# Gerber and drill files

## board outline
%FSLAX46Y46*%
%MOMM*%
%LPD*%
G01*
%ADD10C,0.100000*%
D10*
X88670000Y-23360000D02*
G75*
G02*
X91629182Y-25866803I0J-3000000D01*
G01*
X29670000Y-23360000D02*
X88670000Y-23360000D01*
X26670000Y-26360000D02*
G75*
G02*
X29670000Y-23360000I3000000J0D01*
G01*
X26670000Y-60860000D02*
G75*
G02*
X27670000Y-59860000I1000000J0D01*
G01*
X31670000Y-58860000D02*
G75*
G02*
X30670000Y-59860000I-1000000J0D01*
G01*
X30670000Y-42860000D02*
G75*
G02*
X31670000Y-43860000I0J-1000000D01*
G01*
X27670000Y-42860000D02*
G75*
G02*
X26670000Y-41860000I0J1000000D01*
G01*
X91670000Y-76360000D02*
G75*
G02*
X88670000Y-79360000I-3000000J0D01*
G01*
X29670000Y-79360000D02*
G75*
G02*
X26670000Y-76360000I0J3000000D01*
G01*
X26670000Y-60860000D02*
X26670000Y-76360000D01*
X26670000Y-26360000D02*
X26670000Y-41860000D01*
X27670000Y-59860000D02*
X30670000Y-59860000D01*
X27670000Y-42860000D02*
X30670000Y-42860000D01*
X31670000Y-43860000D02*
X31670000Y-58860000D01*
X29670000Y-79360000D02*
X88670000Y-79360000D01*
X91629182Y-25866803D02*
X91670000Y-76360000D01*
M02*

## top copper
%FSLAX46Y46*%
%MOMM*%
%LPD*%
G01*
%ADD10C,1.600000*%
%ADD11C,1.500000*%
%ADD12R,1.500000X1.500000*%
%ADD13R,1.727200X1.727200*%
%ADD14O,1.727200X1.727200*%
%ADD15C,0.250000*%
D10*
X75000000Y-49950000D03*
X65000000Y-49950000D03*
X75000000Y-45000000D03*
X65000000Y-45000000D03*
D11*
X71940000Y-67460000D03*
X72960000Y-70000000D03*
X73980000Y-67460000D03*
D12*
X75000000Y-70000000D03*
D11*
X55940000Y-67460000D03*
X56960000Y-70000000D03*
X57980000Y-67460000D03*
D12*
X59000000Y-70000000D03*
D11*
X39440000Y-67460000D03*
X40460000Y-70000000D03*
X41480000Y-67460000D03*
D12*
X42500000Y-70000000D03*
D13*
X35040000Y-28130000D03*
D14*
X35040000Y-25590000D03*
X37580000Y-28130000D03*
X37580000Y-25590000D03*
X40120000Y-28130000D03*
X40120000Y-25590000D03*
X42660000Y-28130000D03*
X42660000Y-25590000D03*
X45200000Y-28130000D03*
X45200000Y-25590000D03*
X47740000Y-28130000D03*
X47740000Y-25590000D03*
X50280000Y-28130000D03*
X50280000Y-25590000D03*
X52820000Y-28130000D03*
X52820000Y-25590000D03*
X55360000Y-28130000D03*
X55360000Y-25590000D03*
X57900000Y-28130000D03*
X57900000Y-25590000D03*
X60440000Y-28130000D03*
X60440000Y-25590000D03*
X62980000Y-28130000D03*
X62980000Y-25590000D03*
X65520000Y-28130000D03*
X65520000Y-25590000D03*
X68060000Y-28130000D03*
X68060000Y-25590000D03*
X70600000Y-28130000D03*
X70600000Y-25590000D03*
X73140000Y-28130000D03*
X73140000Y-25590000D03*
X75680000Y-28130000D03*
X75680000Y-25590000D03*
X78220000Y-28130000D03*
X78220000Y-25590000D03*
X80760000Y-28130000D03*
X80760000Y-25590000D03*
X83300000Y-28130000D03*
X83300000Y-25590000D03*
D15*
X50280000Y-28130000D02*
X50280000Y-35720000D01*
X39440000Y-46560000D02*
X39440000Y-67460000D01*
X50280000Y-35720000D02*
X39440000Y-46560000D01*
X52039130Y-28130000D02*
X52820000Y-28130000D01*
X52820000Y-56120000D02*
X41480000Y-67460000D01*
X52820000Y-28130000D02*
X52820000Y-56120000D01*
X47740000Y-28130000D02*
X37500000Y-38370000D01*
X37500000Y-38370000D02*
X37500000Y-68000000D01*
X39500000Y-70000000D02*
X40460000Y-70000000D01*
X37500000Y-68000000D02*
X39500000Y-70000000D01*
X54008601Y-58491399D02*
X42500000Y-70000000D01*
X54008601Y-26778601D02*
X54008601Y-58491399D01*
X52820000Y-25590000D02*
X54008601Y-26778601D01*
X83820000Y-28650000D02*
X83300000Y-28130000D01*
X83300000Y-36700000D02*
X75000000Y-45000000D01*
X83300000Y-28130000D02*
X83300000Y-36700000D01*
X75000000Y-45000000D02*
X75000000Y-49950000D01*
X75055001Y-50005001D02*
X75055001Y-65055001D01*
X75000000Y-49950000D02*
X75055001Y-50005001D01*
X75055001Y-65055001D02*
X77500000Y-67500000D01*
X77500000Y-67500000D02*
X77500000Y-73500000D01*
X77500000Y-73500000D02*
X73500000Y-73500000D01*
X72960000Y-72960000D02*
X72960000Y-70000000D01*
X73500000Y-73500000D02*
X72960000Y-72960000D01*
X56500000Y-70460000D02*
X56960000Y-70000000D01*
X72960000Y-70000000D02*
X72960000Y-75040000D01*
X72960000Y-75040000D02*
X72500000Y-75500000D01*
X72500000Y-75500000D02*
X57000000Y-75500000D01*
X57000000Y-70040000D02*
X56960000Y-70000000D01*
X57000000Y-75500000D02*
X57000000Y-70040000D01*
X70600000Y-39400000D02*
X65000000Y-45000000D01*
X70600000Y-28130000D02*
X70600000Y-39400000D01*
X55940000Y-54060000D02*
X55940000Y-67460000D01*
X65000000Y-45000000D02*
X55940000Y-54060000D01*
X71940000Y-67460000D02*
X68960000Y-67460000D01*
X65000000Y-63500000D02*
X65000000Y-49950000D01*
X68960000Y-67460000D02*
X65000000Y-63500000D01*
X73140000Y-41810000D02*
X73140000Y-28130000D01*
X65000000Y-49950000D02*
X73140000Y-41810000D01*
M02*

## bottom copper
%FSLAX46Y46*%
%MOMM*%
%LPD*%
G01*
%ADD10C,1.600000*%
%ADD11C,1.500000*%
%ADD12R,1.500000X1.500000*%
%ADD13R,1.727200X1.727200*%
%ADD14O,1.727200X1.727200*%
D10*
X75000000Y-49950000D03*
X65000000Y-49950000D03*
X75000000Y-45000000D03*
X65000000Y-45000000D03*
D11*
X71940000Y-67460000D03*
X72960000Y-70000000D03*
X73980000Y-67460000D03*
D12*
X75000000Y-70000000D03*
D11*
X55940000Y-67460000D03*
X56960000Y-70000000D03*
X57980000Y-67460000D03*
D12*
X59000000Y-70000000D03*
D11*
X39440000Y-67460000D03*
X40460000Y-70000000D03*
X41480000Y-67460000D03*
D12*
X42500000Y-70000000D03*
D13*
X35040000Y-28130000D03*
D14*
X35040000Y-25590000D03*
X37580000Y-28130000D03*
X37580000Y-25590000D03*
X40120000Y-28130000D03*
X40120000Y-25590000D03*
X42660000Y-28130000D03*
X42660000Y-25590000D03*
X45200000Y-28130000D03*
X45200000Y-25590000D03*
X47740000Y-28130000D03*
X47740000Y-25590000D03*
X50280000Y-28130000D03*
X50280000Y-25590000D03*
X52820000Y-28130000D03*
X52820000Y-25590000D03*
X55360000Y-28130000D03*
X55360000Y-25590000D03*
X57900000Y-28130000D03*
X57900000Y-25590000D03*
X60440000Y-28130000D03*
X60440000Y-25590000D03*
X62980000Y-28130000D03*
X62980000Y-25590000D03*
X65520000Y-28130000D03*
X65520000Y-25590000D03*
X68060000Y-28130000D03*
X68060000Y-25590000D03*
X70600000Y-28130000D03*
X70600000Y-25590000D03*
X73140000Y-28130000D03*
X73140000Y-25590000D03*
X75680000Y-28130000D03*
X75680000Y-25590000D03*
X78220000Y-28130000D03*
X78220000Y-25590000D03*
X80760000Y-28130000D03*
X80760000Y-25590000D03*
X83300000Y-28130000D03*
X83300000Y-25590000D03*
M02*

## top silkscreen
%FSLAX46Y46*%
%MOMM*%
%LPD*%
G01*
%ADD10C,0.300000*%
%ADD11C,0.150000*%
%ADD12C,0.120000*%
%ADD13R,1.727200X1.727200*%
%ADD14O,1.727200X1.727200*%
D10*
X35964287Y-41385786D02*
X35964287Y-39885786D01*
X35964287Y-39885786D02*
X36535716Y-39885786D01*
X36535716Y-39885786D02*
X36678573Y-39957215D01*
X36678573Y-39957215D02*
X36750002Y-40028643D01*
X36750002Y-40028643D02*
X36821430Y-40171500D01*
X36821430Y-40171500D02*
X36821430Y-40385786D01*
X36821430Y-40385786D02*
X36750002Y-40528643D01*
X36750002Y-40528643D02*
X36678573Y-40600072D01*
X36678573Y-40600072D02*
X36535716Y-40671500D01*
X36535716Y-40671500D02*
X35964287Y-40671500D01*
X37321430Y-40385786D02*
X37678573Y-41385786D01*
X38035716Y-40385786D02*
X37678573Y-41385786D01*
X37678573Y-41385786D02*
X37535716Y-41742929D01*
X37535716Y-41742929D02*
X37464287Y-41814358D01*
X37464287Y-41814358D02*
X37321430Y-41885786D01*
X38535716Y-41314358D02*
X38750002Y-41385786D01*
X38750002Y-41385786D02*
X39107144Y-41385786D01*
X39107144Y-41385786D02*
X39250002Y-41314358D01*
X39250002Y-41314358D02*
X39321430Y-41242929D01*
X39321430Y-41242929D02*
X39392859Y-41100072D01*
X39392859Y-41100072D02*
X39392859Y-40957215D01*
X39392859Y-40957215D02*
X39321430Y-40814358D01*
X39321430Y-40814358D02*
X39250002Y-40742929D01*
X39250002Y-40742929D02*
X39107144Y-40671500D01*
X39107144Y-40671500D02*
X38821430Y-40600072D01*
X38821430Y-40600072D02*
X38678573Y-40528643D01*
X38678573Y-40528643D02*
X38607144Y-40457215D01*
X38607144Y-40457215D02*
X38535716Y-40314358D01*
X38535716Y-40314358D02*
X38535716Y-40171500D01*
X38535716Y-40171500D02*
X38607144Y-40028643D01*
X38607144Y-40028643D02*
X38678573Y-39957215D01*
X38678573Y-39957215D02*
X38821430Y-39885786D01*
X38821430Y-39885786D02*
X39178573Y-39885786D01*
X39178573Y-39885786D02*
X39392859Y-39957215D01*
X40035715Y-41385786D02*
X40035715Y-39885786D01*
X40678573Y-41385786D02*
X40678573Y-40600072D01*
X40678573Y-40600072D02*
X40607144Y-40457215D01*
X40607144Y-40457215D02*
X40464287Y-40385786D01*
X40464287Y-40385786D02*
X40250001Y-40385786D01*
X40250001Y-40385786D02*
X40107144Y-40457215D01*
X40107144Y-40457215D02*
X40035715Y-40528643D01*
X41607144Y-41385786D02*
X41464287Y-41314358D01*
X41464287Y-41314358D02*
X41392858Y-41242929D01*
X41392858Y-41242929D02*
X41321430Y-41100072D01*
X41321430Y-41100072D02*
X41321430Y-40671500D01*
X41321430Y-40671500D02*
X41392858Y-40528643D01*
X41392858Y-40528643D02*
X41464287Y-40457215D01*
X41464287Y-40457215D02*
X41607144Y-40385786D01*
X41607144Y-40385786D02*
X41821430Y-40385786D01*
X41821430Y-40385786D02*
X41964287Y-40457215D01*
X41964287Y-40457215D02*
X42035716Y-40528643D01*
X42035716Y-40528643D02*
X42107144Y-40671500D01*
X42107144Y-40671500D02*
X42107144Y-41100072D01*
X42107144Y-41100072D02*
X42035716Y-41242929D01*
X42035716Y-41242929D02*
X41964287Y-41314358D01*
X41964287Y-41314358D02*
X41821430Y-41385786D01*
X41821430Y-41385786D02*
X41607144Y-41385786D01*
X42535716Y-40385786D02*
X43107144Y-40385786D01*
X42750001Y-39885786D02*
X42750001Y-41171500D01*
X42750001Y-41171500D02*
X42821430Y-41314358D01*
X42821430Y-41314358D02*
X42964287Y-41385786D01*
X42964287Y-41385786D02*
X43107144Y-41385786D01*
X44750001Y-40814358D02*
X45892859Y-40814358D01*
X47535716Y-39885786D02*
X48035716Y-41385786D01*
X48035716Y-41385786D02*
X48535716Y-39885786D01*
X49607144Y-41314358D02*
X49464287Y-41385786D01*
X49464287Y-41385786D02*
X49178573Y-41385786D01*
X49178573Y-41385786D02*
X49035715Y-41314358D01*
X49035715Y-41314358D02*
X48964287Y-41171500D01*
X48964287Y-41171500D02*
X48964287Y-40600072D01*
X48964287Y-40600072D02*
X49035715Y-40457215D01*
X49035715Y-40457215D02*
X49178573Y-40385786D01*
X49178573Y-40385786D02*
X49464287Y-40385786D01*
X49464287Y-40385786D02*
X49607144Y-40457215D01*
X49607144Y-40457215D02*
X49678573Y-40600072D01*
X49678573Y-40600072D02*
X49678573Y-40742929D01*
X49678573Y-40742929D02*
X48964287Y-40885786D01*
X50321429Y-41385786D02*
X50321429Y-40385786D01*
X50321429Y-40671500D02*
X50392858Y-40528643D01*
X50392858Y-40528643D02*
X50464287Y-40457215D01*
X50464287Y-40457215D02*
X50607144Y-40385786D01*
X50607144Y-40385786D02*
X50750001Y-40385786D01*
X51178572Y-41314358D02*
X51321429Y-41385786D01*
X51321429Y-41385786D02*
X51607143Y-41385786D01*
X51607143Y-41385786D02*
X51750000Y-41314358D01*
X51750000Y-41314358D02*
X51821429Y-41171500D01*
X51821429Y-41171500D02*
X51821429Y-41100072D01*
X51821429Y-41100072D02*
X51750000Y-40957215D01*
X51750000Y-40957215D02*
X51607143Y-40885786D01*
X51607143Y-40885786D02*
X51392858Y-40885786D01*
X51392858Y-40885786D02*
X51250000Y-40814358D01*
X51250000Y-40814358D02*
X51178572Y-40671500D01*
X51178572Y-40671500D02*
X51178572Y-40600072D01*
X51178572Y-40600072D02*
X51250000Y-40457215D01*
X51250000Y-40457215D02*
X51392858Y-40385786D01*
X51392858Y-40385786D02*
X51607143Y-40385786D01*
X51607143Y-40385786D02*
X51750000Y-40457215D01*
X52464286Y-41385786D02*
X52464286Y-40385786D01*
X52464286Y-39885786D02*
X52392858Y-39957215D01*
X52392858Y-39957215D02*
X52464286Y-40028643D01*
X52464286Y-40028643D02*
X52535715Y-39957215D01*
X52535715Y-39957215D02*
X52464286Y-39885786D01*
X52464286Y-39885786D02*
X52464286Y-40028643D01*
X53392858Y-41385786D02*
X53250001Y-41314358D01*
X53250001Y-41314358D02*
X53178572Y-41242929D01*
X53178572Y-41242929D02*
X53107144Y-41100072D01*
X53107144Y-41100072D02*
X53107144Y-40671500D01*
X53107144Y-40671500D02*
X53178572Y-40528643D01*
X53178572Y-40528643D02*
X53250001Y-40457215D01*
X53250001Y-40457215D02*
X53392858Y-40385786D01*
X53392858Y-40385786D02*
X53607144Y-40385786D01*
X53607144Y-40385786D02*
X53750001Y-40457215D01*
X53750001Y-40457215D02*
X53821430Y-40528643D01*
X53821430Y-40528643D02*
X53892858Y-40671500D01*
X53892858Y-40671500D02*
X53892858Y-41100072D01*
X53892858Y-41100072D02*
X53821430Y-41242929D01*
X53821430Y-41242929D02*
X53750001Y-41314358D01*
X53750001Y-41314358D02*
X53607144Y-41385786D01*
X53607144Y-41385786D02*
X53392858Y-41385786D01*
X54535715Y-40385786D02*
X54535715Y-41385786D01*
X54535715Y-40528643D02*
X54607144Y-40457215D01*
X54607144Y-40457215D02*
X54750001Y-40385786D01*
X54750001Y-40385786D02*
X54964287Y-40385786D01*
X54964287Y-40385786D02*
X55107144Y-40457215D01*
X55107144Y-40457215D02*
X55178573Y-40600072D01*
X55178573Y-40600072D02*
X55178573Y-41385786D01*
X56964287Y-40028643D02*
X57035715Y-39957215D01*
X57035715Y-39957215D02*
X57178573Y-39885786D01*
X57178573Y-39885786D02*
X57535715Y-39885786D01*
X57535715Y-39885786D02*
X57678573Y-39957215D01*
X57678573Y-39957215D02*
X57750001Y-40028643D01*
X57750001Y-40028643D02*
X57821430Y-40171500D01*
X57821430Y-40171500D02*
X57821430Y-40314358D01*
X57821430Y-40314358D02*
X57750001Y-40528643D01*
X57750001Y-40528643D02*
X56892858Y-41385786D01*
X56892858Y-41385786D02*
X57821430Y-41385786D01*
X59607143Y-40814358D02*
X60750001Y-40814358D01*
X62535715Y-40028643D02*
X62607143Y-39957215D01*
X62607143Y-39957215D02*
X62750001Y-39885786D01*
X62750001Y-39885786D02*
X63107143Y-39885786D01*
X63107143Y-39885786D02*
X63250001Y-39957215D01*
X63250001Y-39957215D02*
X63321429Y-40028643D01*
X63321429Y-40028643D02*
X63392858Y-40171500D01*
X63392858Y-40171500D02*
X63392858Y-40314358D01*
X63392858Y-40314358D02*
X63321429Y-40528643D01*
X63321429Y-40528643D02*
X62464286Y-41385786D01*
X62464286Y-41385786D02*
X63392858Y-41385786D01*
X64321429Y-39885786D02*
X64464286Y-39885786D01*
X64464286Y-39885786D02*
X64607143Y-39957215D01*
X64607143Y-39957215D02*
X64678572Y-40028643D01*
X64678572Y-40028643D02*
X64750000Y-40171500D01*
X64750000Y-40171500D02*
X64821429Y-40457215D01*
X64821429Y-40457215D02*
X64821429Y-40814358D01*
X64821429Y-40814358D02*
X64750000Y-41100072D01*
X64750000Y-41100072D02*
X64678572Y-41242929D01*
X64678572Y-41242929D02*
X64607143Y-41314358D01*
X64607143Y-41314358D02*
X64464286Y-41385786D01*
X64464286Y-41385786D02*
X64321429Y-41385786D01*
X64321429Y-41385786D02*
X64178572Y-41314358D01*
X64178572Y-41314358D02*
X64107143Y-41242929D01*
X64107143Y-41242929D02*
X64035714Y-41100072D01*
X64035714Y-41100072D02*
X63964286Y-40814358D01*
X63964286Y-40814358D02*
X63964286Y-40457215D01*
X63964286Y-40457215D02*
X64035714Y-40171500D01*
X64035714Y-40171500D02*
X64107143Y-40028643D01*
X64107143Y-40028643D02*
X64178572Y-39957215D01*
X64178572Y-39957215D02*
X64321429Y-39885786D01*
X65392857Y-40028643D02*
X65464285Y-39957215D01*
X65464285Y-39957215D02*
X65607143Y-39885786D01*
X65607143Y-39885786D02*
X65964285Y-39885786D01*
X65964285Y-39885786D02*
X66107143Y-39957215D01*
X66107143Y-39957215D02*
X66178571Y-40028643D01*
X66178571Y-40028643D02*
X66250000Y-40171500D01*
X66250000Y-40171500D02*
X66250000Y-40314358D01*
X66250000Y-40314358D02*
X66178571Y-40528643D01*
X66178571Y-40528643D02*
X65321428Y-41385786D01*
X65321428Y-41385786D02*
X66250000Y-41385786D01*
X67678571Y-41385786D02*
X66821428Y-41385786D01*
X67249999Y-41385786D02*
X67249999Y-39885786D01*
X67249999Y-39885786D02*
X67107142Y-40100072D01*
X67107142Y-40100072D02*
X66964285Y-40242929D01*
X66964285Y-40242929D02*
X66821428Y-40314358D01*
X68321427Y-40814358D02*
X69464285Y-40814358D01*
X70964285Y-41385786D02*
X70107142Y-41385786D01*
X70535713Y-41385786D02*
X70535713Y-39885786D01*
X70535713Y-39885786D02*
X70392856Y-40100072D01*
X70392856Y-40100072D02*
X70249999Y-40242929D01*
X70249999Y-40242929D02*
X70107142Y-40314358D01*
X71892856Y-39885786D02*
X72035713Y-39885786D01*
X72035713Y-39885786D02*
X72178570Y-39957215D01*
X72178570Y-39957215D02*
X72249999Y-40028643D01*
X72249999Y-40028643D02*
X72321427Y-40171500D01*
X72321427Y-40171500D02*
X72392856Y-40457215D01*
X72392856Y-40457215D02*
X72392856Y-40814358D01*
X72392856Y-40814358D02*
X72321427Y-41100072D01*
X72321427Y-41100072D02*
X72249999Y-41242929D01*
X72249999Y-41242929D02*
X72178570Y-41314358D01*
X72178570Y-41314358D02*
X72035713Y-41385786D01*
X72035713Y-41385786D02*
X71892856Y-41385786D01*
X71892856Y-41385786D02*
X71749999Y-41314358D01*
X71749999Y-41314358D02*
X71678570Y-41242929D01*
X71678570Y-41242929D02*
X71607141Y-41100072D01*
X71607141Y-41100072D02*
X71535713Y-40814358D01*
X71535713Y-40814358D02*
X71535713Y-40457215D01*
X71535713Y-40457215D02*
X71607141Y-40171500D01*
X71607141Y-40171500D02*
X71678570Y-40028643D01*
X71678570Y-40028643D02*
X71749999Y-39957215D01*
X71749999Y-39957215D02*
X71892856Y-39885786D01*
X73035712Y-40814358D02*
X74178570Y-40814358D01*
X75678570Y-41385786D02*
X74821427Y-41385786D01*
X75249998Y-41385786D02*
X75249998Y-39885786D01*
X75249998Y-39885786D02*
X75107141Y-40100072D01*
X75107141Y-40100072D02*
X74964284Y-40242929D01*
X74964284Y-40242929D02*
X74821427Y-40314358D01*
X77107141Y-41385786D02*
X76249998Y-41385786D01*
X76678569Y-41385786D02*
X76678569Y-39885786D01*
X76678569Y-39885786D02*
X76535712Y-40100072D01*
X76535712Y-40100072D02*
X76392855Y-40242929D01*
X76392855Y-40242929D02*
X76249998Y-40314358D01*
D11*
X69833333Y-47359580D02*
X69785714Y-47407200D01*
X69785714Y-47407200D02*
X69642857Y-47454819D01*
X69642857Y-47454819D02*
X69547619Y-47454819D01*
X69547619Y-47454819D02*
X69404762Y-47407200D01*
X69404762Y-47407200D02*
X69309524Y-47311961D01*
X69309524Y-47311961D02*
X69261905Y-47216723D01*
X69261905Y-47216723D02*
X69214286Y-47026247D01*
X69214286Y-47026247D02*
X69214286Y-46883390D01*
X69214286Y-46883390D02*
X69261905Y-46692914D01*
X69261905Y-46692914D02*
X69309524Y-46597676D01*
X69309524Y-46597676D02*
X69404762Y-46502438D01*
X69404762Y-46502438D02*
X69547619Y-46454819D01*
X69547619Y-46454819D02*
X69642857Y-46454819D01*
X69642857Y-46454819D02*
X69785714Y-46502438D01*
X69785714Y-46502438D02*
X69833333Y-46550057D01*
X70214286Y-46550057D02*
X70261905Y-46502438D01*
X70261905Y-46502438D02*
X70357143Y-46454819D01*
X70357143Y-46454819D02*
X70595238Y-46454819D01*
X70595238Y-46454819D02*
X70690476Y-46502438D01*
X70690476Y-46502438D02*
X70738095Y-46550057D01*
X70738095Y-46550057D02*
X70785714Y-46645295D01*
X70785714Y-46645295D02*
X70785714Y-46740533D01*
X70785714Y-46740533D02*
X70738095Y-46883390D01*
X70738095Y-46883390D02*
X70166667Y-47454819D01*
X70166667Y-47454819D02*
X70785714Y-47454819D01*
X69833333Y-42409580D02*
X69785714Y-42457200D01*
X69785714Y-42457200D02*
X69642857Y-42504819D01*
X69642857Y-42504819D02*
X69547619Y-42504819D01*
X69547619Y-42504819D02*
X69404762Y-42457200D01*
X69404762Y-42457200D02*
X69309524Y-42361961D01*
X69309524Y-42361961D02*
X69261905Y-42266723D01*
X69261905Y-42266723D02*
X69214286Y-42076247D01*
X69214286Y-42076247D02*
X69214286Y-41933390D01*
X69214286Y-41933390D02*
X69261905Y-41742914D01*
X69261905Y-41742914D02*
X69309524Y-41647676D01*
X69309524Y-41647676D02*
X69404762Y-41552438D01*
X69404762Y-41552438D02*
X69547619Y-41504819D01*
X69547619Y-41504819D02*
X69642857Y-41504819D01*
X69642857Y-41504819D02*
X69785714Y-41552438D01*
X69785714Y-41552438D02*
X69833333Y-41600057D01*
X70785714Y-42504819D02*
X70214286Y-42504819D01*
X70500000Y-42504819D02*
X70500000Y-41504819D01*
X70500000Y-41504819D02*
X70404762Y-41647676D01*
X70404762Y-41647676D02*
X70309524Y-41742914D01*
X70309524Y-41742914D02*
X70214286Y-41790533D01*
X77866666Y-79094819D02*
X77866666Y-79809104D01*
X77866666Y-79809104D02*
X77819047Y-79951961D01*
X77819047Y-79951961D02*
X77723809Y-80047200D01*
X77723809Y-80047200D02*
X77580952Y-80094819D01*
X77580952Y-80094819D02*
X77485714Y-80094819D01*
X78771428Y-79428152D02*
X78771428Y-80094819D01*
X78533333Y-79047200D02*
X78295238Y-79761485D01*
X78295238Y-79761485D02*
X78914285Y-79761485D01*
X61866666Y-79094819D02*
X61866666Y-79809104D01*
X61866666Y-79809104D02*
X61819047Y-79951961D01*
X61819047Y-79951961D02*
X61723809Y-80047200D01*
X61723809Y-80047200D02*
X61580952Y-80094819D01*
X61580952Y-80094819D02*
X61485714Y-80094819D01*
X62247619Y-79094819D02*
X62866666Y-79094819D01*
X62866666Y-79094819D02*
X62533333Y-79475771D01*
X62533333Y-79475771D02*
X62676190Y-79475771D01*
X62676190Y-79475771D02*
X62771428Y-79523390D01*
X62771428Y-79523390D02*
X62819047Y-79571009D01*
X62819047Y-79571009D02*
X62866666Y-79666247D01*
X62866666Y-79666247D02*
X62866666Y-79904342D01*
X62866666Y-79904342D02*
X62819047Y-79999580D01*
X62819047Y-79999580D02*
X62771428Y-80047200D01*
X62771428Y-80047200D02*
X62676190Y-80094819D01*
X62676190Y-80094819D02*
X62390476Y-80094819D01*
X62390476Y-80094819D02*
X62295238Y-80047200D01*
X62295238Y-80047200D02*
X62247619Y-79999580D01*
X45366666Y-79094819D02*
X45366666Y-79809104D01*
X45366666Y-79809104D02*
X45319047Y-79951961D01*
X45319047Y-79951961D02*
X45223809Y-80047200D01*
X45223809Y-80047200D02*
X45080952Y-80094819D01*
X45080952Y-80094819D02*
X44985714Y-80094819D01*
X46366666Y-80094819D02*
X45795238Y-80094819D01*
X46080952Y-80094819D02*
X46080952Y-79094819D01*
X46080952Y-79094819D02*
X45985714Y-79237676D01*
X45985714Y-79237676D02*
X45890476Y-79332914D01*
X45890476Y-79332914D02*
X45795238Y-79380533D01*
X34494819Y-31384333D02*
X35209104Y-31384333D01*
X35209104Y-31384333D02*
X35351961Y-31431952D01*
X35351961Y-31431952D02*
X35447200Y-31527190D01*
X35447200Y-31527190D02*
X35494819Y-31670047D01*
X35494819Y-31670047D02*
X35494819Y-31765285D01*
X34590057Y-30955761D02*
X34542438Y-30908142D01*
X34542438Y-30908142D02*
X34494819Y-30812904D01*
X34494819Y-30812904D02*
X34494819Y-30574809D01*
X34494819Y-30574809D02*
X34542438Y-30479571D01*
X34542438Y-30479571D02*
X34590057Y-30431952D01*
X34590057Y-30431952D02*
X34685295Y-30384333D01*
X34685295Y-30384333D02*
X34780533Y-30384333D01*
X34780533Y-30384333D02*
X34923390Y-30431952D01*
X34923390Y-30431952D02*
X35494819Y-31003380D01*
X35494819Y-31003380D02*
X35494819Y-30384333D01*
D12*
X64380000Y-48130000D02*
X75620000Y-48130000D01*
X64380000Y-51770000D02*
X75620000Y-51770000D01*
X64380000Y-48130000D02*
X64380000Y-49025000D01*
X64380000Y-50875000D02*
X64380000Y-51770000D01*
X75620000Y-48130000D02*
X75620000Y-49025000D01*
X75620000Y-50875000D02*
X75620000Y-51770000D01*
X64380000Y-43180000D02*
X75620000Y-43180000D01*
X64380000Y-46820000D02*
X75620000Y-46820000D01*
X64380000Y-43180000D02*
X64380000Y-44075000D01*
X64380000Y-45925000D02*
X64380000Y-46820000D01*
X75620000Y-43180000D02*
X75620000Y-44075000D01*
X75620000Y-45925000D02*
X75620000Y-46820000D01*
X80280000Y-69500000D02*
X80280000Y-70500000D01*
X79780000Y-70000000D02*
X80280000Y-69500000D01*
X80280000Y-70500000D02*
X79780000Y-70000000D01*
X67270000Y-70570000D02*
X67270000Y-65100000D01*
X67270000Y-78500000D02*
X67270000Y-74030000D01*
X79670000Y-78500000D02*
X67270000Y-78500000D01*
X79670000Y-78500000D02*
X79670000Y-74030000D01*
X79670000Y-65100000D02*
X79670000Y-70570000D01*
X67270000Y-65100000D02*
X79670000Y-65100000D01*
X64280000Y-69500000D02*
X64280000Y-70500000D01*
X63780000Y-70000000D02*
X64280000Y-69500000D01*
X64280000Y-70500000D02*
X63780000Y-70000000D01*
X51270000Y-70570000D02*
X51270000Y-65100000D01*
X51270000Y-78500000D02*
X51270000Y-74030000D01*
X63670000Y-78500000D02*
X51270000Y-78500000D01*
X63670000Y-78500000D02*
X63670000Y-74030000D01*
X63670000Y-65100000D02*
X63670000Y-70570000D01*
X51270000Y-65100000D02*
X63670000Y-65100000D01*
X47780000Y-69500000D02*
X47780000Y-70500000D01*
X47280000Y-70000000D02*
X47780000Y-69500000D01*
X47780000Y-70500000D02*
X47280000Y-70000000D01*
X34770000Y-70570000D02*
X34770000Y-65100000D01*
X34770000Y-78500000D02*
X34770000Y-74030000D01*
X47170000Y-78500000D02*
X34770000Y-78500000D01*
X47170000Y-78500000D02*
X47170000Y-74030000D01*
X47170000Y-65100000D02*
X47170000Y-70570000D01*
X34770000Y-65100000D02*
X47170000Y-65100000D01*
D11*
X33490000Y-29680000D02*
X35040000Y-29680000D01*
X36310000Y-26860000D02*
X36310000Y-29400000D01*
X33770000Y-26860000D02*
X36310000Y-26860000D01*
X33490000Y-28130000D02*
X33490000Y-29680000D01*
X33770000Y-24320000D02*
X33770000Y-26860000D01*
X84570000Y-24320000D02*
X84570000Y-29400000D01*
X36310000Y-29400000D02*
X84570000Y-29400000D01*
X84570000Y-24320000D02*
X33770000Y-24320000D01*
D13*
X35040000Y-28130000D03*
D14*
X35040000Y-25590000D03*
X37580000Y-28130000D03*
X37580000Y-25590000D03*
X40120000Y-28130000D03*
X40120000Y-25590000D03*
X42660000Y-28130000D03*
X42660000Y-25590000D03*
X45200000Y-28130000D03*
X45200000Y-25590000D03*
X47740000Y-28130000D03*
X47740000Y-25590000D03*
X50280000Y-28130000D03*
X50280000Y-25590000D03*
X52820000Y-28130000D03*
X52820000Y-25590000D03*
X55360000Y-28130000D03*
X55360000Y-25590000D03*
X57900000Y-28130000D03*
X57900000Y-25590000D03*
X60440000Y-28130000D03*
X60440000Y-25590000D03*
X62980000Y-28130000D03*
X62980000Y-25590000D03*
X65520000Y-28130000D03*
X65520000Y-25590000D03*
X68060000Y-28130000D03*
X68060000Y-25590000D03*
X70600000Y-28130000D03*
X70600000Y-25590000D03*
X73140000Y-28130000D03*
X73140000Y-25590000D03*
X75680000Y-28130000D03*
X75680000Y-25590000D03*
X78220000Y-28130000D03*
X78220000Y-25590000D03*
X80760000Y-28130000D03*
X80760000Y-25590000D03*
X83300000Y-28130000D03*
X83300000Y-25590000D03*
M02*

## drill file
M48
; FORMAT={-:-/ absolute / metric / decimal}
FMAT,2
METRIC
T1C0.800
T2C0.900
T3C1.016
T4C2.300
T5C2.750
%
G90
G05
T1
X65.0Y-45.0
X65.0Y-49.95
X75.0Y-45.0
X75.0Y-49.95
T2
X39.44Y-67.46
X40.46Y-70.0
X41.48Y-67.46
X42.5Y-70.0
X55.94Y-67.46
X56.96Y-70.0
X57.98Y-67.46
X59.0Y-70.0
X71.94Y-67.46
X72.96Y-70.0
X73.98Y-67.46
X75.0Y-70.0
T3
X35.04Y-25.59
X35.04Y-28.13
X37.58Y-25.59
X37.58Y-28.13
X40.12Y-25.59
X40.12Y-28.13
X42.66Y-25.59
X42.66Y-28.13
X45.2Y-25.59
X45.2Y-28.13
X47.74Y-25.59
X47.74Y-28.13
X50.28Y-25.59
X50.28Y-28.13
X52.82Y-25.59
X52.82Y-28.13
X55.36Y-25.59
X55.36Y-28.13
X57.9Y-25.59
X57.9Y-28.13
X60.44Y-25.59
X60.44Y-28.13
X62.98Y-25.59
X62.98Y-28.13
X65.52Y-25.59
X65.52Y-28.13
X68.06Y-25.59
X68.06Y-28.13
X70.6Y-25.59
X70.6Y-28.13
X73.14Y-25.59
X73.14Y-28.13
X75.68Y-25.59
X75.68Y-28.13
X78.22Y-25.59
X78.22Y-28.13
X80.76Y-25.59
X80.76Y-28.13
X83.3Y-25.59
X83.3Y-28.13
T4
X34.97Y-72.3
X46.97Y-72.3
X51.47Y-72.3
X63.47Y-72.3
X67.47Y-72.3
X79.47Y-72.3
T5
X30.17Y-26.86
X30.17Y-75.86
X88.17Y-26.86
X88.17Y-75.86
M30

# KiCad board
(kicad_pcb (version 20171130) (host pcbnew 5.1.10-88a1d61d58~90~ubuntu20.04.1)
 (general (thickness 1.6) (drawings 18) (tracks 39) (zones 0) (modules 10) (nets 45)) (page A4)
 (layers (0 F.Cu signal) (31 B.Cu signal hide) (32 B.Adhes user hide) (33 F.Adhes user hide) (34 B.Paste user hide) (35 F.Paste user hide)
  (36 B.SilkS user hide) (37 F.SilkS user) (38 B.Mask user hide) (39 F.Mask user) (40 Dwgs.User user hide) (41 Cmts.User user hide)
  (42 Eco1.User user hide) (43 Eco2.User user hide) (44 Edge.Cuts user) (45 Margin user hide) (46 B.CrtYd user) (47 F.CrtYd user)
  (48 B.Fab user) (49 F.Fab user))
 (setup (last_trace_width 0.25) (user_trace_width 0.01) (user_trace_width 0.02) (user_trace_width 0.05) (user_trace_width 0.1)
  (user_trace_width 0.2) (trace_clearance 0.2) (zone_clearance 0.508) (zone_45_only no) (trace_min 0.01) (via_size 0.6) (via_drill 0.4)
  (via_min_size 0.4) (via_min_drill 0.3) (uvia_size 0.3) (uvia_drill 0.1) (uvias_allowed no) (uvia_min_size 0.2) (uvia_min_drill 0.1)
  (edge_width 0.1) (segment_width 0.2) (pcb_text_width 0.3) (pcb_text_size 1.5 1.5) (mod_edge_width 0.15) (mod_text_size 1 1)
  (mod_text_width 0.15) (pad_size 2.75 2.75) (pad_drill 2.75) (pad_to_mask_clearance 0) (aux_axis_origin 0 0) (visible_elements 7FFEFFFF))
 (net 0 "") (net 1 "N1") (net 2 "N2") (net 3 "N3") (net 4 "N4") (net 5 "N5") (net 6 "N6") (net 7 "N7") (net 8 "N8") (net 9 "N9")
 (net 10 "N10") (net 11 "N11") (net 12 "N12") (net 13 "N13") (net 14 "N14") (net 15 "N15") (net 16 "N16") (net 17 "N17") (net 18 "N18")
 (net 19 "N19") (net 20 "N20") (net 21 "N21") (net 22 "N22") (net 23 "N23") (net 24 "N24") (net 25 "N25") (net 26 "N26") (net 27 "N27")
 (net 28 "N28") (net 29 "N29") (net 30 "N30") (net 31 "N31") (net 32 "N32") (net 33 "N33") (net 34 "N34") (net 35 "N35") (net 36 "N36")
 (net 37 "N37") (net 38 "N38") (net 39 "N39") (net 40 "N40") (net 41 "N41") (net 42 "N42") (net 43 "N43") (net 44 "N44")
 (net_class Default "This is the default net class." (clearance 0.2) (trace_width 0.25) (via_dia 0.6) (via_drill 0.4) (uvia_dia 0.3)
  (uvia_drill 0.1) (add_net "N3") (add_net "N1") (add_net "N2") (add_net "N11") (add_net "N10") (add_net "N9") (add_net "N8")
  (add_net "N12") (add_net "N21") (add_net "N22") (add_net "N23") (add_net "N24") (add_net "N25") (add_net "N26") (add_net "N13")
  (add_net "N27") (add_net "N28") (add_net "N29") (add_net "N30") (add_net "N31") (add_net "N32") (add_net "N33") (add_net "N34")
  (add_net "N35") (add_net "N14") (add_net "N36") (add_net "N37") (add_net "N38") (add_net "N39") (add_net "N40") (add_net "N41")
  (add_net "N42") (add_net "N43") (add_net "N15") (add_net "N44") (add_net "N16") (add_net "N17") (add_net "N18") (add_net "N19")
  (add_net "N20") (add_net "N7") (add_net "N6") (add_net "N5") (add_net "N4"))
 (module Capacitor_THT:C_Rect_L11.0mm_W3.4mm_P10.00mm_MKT (layer F.Cu) (at 65 49.95)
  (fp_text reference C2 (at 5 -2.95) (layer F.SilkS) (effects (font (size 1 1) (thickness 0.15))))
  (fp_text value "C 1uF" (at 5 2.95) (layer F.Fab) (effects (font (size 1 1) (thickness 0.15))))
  (fp_line (start -0.62 -1.82) (end 10.62 -1.82) (layer F.SilkS) (width 0.12))
  (fp_line (start -0.62 1.82) (end 10.62 1.82) (layer F.SilkS) (width 0.12))
  (fp_line (start -0.62 -1.82) (end -0.62 -0.925) (layer F.SilkS) (width 0.12))
  (fp_line (start -0.62 0.925) (end -0.62 1.82) (layer F.SilkS) (width 0.12))
  (fp_line (start 10.62 -1.82) (end 10.62 -0.925) (layer F.SilkS) (width 0.12))
  (fp_line (start 10.62 0.925) (end 10.62 1.82) (layer F.SilkS) (width 0.12))
  (pad 2 thru_hole circle (at 10 0) (size 1.6 1.6) (drill 0.8) (layers *.Cu *.Mask) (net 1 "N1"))
  (pad 1 thru_hole circle (at 0 0) (size 1.6 1.6) (drill 0.8) (layers *.Cu *.Mask) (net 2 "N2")))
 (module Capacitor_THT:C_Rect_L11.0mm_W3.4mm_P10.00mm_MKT (layer F.Cu) (at 65 45)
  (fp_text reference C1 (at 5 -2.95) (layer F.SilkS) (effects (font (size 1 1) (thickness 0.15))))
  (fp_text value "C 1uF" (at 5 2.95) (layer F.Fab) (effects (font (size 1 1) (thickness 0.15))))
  (fp_line (start -0.62 -1.82) (end 10.62 -1.82) (layer F.SilkS) (width 0.12))
  (fp_line (start -0.62 1.82) (end 10.62 1.82) (layer F.SilkS) (width 0.12))
  (fp_line (start -0.62 -1.82) (end -0.62 -0.925) (layer F.SilkS) (width 0.12))
  (fp_line (start -0.62 0.925) (end -0.62 1.82) (layer F.SilkS) (width 0.12))
  (fp_line (start 10.62 -1.82) (end 10.62 -0.925) (layer F.SilkS) (width 0.12))
  (fp_line (start 10.62 0.925) (end 10.62 1.82) (layer F.SilkS) (width 0.12))
  (pad 2 thru_hole circle (at 10 0) (size 1.6 1.6) (drill 0.8) (layers *.Cu *.Mask) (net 1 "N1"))
  (pad 1 thru_hole circle (at 0 0) (size 1.6 1.6) (drill 0.8) (layers *.Cu *.Mask) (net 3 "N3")))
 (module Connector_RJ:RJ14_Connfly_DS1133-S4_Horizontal (layer F.Cu) (at 75 70 180)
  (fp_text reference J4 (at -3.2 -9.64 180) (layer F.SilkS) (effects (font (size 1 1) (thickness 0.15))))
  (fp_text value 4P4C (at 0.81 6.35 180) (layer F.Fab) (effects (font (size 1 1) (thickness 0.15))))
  (fp_line (start -5.28 0.5) (end -5.28 -0.5) (layer F.SilkS) (width 0.12))
  (fp_line (start -4.78 0) (end -5.28 0.5) (layer F.SilkS) (width 0.12))
  (fp_line (start -5.28 -0.5) (end -4.78 0) (layer F.SilkS) (width 0.12))
  (fp_line (start 7.73 -0.57) (end 7.73 4.9) (layer F.SilkS) (width 0.12))
  (fp_line (start 7.73 -8.5) (end 7.73 -4.03) (layer F.SilkS) (width 0.12))
  (fp_line (start -4.67 -8.5) (end 7.73 -8.5) (layer F.SilkS) (width 0.12))
  (fp_line (start -4.67 -8.5) (end -4.67 -4.03) (layer F.SilkS) (width 0.12))
  (fp_line (start -4.67 4.9) (end -4.67 -0.57) (layer F.SilkS) (width 0.12))
  (fp_line (start 7.73 4.9) (end -4.67 4.9) (layer F.SilkS) (width 0.12))
  (pad 4 thru_hole circle (at 3.06 2.54) (size 1.5 1.5) (drill 0.9) (layers *.Cu *.Mask) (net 2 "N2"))
  (pad "" np_thru_hole circle (at 7.53 -2.3) (size 2.3 2.3) (drill 2.3) (layers *.Cu *.Mask))
  (pad 3 thru_hole circle (at 2.04 0) (size 1.5 1.5) (drill 0.9) (layers *.Cu *.Mask) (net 1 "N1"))
  (pad 2 thru_hole circle (at 1.02 2.54) (size 1.5 1.5) (drill 0.9) (layers *.Cu *.Mask) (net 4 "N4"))
  (pad 1 thru_hole rect (at 0 0) (size 1.5 1.5) (drill 0.9) (layers *.Cu *.Mask) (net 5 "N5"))
  (pad "" np_thru_hole circle (at -4.47 -2.3) (size 2.3 2.3) (drill 2.3) (layers *.Cu *.Mask)))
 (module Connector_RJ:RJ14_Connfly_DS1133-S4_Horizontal (layer F.Cu) (at 59 70 180)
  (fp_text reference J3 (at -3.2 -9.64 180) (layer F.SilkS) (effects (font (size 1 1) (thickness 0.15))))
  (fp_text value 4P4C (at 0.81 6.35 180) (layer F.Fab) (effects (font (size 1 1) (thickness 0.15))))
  (fp_line (start -5.28 0.5) (end -5.28 -0.5) (layer F.SilkS) (width 0.12))
  (fp_line (start -4.78 0) (end -5.28 0.5) (layer F.SilkS) (width 0.12))
  (fp_line (start -5.28 -0.5) (end -4.78 0) (layer F.SilkS) (width 0.12))
  (fp_line (start 7.73 -0.57) (end 7.73 4.9) (layer F.SilkS) (width 0.12))
  (fp_line (start 7.73 -8.5) (end 7.73 -4.03) (layer F.SilkS) (width 0.12))
  (fp_line (start -4.67 -8.5) (end 7.73 -8.5) (layer F.SilkS) (width 0.12))
  (fp_line (start -4.67 -8.5) (end -4.67 -4.03) (layer F.SilkS) (width 0.12))
  (fp_line (start -4.67 4.9) (end -4.67 -0.57) (layer F.SilkS) (width 0.12))
  (fp_line (start 7.73 4.9) (end -4.67 4.9) (layer F.SilkS) (width 0.12))
  (pad 4 thru_hole circle (at 3.06 2.54) (size 1.5 1.5) (drill 0.9) (layers *.Cu *.Mask) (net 3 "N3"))
  (pad "" np_thru_hole circle (at 7.53 -2.3) (size 2.3 2.3) (drill 2.3) (layers *.Cu *.Mask))
  (pad 3 thru_hole circle (at 2.04 0) (size 1.5 1.5) (drill 0.9) (layers *.Cu *.Mask) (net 1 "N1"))
  (pad 2 thru_hole circle (at 1.02 2.54) (size 1.5 1.5) (drill 0.9) (layers *.Cu *.Mask) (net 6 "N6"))
  (pad 1 thru_hole rect (at 0 0) (size 1.5 1.5) (drill 0.9) (layers *.Cu *.Mask) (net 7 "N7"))
  (pad "" np_thru_hole circle (at -4.47 -2.3) (size 2.3 2.3) (drill 2.3) (layers *.Cu *.Mask)))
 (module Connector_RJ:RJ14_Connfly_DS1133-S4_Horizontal (layer F.Cu) (at 42.5 70 180)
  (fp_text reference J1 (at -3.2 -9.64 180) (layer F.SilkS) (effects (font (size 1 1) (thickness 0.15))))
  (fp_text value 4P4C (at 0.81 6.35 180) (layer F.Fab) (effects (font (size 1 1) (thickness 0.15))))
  (fp_line (start -5.28 0.5) (end -5.28 -0.5) (layer F.SilkS) (width 0.12))
  (fp_line (start -4.78 0) (end -5.28 0.5) (layer F.SilkS) (width 0.12))
  (fp_line (start -5.28 -0.5) (end -4.78 0) (layer F.SilkS) (width 0.12))
  (fp_line (start 7.73 -0.57) (end 7.73 4.9) (layer F.SilkS) (width 0.12))
  (fp_line (start 7.73 -8.5) (end 7.73 -4.03) (layer F.SilkS) (width 0.12))
  (fp_line (start -4.67 -8.5) (end 7.73 -8.5) (layer F.SilkS) (width 0.12))
  (fp_line (start -4.67 -8.5) (end -4.67 -4.03) (layer F.SilkS) (width 0.12))
  (fp_line (start -4.67 4.9) (end -4.67 -0.57) (layer F.SilkS) (width 0.12))
  (fp_line (start 7.73 4.9) (end -4.67 4.9) (layer F.SilkS) (width 0.12))
  (pad 4 thru_hole circle (at 3.06 2.54) (size 1.5 1.5) (drill 0.9) (layers *.Cu *.Mask) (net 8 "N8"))
  (pad "" np_thru_hole circle (at 7.53 -2.3) (size 2.3 2.3) (drill 2.3) (layers *.Cu *.Mask))
  (pad 3 thru_hole circle (at 2.04 0) (size 1.5 1.5) (drill 0.9) (layers *.Cu *.Mask) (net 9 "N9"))
  (pad 2 thru_hole circle (at 1.02 2.54) (size 1.5 1.5) (drill 0.9) (layers *.Cu *.Mask) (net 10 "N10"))
  (pad 1 thru_hole rect (at 0 0) (size 1.5 1.5) (drill 0.9) (layers *.Cu *.Mask) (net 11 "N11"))
  (pad "" np_thru_hole circle (at -4.47 -2.3) (size 2.3 2.3) (drill 2.3) (layers *.Cu *.Mask)))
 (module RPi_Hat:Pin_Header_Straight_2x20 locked (layer F.Cu) (at 59.17 26.86 90)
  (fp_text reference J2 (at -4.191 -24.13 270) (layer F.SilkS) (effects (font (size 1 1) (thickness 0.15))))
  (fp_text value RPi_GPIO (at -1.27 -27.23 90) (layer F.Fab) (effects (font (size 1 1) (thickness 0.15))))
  (fp_line (start -2.82 -25.68) (end -2.82 -24.13) (layer F.SilkS) (width 0.15))
  (fp_line (start 0 -22.86) (end -2.54 -22.86) (layer F.SilkS) (width 0.15))
  (fp_line (start 0 -25.4) (end 0 -22.86) (layer F.SilkS) (width 0.15))
  (fp_line (start -1.27 -25.68) (end -2.82 -25.68) (layer F.SilkS) (width 0.15))
  (fp_line (start 2.54 -25.4) (end 0 -25.4) (layer F.SilkS) (width 0.15))
  (fp_line (start 2.54 25.4) (end -2.54 25.4) (layer F.SilkS) (width 0.15))
  (fp_line (start -2.54 -22.86) (end -2.54 25.4) (layer F.SilkS) (width 0.15))
  (fp_line (start 2.54 25.4) (end 2.54 -25.4) (layer F.SilkS) (width 0.15))
  (pad 1 thru_hole rect (at -1.27 -24.13 90) (size 1.7272 1.7272) (drill 1.016) (layers *.Cu *.Mask F.SilkS) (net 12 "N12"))
  (pad 2 thru_hole oval (at 1.27 -24.13 90) (size 1.7272 1.7272) (drill 1.016) (layers *.Cu *.Mask F.SilkS) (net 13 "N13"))
  (pad 3 thru_hole oval (at -1.27 -21.59 90) (size 1.7272 1.7272) (drill 1.016) (layers *.Cu *.Mask F.SilkS) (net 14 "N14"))
  (pad 4 thru_hole oval (at 1.27 -21.59 90) (size 1.7272 1.7272) (drill 1.016) (layers *.Cu *.Mask F.SilkS) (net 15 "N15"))
  (pad 5 thru_hole oval (at -1.27 -19.05 90) (size 1.7272 1.7272) (drill 1.016) (layers *.Cu *.Mask F.SilkS) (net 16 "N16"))
  (pad 6 thru_hole oval (at 1.27 -19.05 90) (size 1.7272 1.7272) (drill 1.016) (layers *.Cu *.Mask F.SilkS) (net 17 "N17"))
  (pad 7 thru_hole oval (at -1.27 -16.51 90) (size 1.7272 1.7272) (drill 1.016) (layers *.Cu *.Mask F.SilkS) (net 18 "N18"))
  (pad 8 thru_hole oval (at 1.27 -16.51 90) (size 1.7272 1.7272) (drill 1.016) (layers *.Cu *.Mask F.SilkS) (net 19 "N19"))
  (pad 9 thru_hole oval (at -1.27 -13.97 90) (size 1.7272 1.7272) (drill 1.016) (layers *.Cu *.Mask F.SilkS) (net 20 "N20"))
  (pad 10 thru_hole oval (at 1.27 -13.97 90) (size 1.7272 1.7272) (drill 1.016) (layers *.Cu *.Mask F.SilkS) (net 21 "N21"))
  (pad 11 thru_hole oval (at -1.27 -11.43 90) (size 1.7272 1.7272) (drill 1.016) (layers *.Cu *.Mask F.SilkS) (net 9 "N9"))
  (pad 12 thru_hole oval (at 1.27 -11.43 90) (size 1.7272 1.7272) (drill 1.016) (layers *.Cu *.Mask F.SilkS) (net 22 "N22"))
  (pad 13 thru_hole oval (at -1.27 -8.89 90) (size 1.7272 1.7272) (drill 1.016) (layers *.Cu *.Mask F.SilkS) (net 8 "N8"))
  (pad 14 thru_hole oval (at 1.27 -8.89 90) (size 1.7272 1.7272) (drill 1.016) (layers *.Cu *.Mask F.SilkS) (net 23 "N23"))
  (pad 15 thru_hole oval (at -1.27 -6.35 90) (size 1.7272 1.7272) (drill 1.016) (layers *.Cu *.Mask F.SilkS) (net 10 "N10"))
  (pad 16 thru_hole oval (at 1.27 -6.35 90) (size 1.7272 1.7272) (drill 1.016) (layers *.Cu *.Mask F.SilkS) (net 11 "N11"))
  (pad 17 thru_hole oval (at -1.27 -3.81 90) (size 1.7272 1.7272) (drill 1.016) (layers *.Cu *.Mask F.SilkS) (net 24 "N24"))
  (pad 18 thru_hole oval (at 1.27 -3.81 90) (size 1.7272 1.7272) (drill 1.016) (layers *.Cu *.Mask F.SilkS) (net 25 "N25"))
  (pad 19 thru_hole oval (at -1.27 -1.27 90) (size 1.7272 1.7272) (drill 1.016) (layers *.Cu *.Mask F.SilkS) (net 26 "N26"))
  (pad 20 thru_hole oval (at 1.27 -1.27 90) (size 1.7272 1.7272) (drill 1.016) (layers *.Cu *.Mask F.SilkS) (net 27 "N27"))
  (pad 21 thru_hole oval (at -1.27 1.27 90) (size 1.7272 1.7272) (drill 1.016) (layers *.Cu *.Mask F.SilkS) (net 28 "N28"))
  (pad 22 thru_hole oval (at 1.27 1.27 90) (size 1.7272 1.7272) (drill 1.016) (layers *.Cu *.Mask F.SilkS) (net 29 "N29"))
  (pad 23 thru_hole oval (at -1.27 3.81 90) (size 1.7272 1.7272) (drill 1.016) (layers *.Cu *.Mask F.SilkS) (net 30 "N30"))
  (pad 24 thru_hole oval (at 1.27 3.81 90) (size 1.7272 1.7272) (drill 1.016) (layers *.Cu *.Mask F.SilkS) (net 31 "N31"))
  (pad 25 thru_hole oval (at -1.27 6.35 90) (size 1.7272 1.7272) (drill 1.016) (layers *.Cu *.Mask F.SilkS) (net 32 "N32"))
  (pad 26 thru_hole oval (at 1.27 6.35 90) (size 1.7272 1.7272) (drill 1.016) (layers *.Cu *.Mask F.SilkS) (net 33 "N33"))
  (pad 27 thru_hole oval (at -1.27 8.89 90) (size 1.7272 1.7272) (drill 1.016) (layers *.Cu *.Mask F.SilkS) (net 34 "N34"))
  (pad 28 thru_hole oval (at 1.27 8.89 90) (size 1.7272 1.7272) (drill 1.016) (layers *.Cu *.Mask F.SilkS) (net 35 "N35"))
  (pad 29 thru_hole oval (at -1.27 11.43 90) (size 1.7272 1.7272) (drill 1.016) (layers *.Cu *.Mask F.SilkS) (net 3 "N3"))
  (pad 30 thru_hole oval (at 1.27 11.43 90) (size 1.7272 1.7272) (drill 1.016) (layers *.Cu *.Mask F.SilkS) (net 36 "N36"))
  (pad 31 thru_hole oval (at -1.27 13.97 90) (size 1.7272 1.7272) (drill 1.016) (layers *.Cu *.Mask F.SilkS) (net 2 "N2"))
  (pad 32 thru_hole oval (at 1.27 13.97 90) (size 1.7272 1.7272) (drill 1.016) (layers *.Cu *.Mask F.SilkS) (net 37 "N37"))
  (pad 33 thru_hole oval (at -1.27 16.51 90) (size 1.7272 1.7272) (drill 1.016) (layers *.Cu *.Mask F.SilkS) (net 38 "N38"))
  (pad 34 thru_hole oval (at 1.27 16.51 90) (size 1.7272 1.7272) (drill 1.016) (layers *.Cu *.Mask F.SilkS) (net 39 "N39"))
  (pad 35 thru_hole oval (at -1.27 19.05 90) (size 1.7272 1.7272) (drill 1.016) (layers *.Cu *.Mask F.SilkS) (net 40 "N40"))
  (pad 36 thru_hole oval (at 1.27 19.05 90) (size 1.7272 1.7272) (drill 1.016) (layers *.Cu *.Mask F.SilkS) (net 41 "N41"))
  (pad 37 thru_hole oval (at -1.27 21.59 90) (size 1.7272 1.7272) (drill 1.016) (layers *.Cu *.Mask F.SilkS) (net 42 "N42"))
  (pad 38 thru_hole oval (at 1.27 21.59 90) (size 1.7272 1.7272) (drill 1.016) (layers *.Cu *.Mask F.SilkS) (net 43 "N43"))
  (pad 39 thru_hole oval (at -1.27 24.13 90) (size 1.7272 1.7272) (drill 1.016) (layers *.Cu *.Mask F.SilkS) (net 1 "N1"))
  (pad 40 thru_hole oval (at 1.27 24.13 90) (size 1.7272 1.7272) (drill 1.016) (layers *.Cu *.Mask F.SilkS) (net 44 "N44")))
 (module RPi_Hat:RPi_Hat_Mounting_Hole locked (layer F.Cu) (at 88.17 26.86)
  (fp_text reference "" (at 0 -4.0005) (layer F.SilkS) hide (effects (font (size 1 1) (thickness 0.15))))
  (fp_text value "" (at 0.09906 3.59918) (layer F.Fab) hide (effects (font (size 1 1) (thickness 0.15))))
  (pad "" np_thru_hole circle (at 0 0) (size 2.75 2.75) (drill 2.75) (layers *.Cu *.Mask) (solder_mask_margin 1.725) (clearance 1.725)))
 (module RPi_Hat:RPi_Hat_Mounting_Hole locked (layer F.Cu) (at 88.17 75.86)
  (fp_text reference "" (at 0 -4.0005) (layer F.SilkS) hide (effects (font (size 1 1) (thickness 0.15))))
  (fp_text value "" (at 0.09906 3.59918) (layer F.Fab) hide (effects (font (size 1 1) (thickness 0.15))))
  (pad "" np_thru_hole circle (at 0 0) (size 2.75 2.75) (drill 2.75) (layers *.Cu *.Mask) (solder_mask_margin 1.725) (clearance 1.725)))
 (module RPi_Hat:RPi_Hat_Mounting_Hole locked (layer F.Cu) (at 30.17 75.86)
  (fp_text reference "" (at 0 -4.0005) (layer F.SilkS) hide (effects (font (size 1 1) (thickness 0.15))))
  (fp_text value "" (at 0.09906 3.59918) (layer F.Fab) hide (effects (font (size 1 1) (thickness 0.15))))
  (pad "" np_thru_hole circle (at 0 0) (size 2.75 2.75) (drill 2.75) (layers *.Cu *.Mask) (solder_mask_margin 1.725) (clearance 1.725)))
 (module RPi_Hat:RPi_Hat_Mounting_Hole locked (layer F.Cu) (at 30.17 26.86)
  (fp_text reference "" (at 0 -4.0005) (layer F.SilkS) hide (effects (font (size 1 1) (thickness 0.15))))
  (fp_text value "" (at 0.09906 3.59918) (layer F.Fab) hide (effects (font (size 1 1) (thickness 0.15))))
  (pad "" np_thru_hole circle (at 0 0) (size 2.75 2.75) (drill 2.75) (layers *.Cu *.Mask) (solder_mask_margin 1.725) (clearance 1.725)))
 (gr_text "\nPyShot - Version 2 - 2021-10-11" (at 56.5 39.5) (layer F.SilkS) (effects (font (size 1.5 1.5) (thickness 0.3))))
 (gr_arc (start 88.67 26.36) (end 88.67 23.36) (angle 80.53767779) (layer Edge.Cuts) (width 0.1))
 (gr_line (start 29.67 23.36) (end 88.67 23.36) (angle 90) (layer Edge.Cuts) (width 0.1))
 (gr_arc (start 29.67 26.36) (end 26.67 26.36) (angle 90) (layer Edge.Cuts) (width 0.1))
 (gr_arc (start 27.67 60.86) (end 26.67 60.86) (angle 90) (layer Edge.Cuts) (width 0.1))
 (gr_arc (start 30.67 58.86) (end 31.67 58.86) (angle 90) (layer Edge.Cuts) (width 0.1))
 (gr_arc (start 30.67 43.86) (end 30.67 42.86) (angle 90) (layer Edge.Cuts) (width 0.1))
 (gr_arc (start 27.67 41.86) (end 27.67 42.86) (angle 90) (layer Edge.Cuts) (width 0.1))
 (gr_arc (start 88.67 76.36) (end 91.67 76.36) (angle 90) (layer Edge.Cuts) (width 0.1))
 (gr_arc (start 29.67 76.36) (end 29.67 79.36) (angle 90) (layer Edge.Cuts) (width 0.1))
 (gr_line (start 26.67 60.86) (end 26.67 76.36) (layer Edge.Cuts) (width 0.1))
 (gr_line (start 26.67 26.36) (end 26.67 41.86) (layer Edge.Cuts) (width 0.1))
 (gr_line (start 27.67 59.86) (end 30.67 59.86) (layer Edge.Cuts) (width 0.1))
 (gr_line (start 27.67 42.86) (end 30.67 42.86) (layer Edge.Cuts) (width 0.1))
 (gr_line (start 31.67 43.86) (end 31.67 58.86) (layer Edge.Cuts) (width 0.1))
 (gr_line (start 29.67 79.36) (end 88.67 79.36) (angle 90) (layer Edge.Cuts) (width 0.1))
 (gr_line (start 91.629182 25.866803) (end 91.67 76.36) (angle 90) (layer Edge.Cuts) (width 0.1))
 (segment (start 50.28 28.13) (end 50.28 35.72) (width 0.25) (layer F.Cu) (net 8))
 (segment (start 39.44 46.56) (end 39.44 67.46) (width 0.25) (layer F.Cu) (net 8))
 (segment (start 50.28 35.72) (end 39.44 46.56) (width 0.25) (layer F.Cu) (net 8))
 (segment (start 52.03913 28.13) (end 52.82 28.13) (width 0.25) (layer F.Cu) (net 10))
 (segment (start 52.82 56.12) (end 41.48 67.46) (width 0.25) (layer F.Cu) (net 10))
 (segment (start 52.82 28.13) (end 52.82 56.12) (width 0.25) (layer F.Cu) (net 10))
 (segment (start 47.74 28.13) (end 37.5 38.37) (width 0.25) (layer F.Cu) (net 9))
 (segment (start 37.5 38.37) (end 37.5 68) (width 0.25) (layer F.Cu) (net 9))
 (segment (start 39.5 70) (end 40.46 70) (width 0.25) (layer F.Cu) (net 9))
 (segment (start 37.5 68) (end 39.5 70) (width 0.25) (layer F.Cu) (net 9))
 (segment (start 54.008601 58.491399) (end 42.5 70) (width 0.25) (layer F.Cu) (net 11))
 (segment (start 54.008601 26.778601) (end 54.008601 58.491399) (width 0.25) (layer F.Cu) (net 11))
 (segment (start 52.82 25.59) (end 54.008601 26.778601) (width 0.25) (layer F.Cu) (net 11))
 (segment (start 83.82 28.65) (end 83.3 28.13) (width 0.25) (layer F.Cu) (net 1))
 (segment (start 83.3 36.7) (end 75 45) (width 0.25) (layer F.Cu) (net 1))
 (segment (start 83.3 28.13) (end 83.3 36.7) (width 0.25) (layer F.Cu) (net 1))
 (segment (start 75 45) (end 75 49.95) (width 0.25) (layer F.Cu) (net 1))
 (segment (start 75.055001 50.005001) (end 75.055001 65.055001) (width 0.25) (layer F.Cu) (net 1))
 (segment (start 75 49.95) (end 75.055001 50.005001) (width 0.25) (layer F.Cu) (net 1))
 (segment (start 75.055001 65.055001) (end 77.5 67.5) (width 0.25) (layer F.Cu) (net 1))
 (segment (start 77.5 67.5) (end 77.5 73.5) (width 0.25) (layer F.Cu) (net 1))
 (segment (start 77.5 73.5) (end 73.5 73.5) (width 0.25) (layer F.Cu) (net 1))
 (segment (start 72.96 72.96) (end 72.96 70) (width 0.25) (layer F.Cu) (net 1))
 (segment (start 73.5 73.5) (end 72.96 72.96) (width 0.25) (layer F.Cu) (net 1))
 (segment (start 56.5 70.46) (end 56.96 70) (width 0.25) (layer F.Cu) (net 1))
 (segment (start 72.96 70) (end 72.96 75.04) (width 0.25) (layer F.Cu) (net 1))
 (segment (start 72.96 75.04) (end 72.5 75.5) (width 0.25) (layer F.Cu) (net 1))
 (segment (start 72.5 75.5) (end 57 75.5) (width 0.25) (layer F.Cu) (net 1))
 (segment (start 57 70.04) (end 56.96 70) (width 0.25) (layer F.Cu) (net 1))
 (segment (start 57 75.5) (end 57 70.04) (width 0.25) (layer F.Cu) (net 1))
 (segment (start 70.6 39.4) (end 65 45) (width 0.25) (layer F.Cu) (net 3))
 (segment (start 70.6 28.13) (end 70.6 39.4) (width 0.25) (layer F.Cu) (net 3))
 (segment (start 55.94 54.06) (end 55.94 67.46) (width 0.25) (layer F.Cu) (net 3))
 (segment (start 65 45) (end 55.94 54.06) (width 0.25) (layer F.Cu) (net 3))
 (segment (start 71.94 67.46) (end 68.96 67.46) (width 0.25) (layer F.Cu) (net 2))
 (segment (start 65 63.5) (end 65 49.95) (width 0.25) (layer F.Cu) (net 2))
 (segment (start 68.96 67.46) (end 65 63.5) (width 0.25) (layer F.Cu) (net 2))
 (segment (start 73.14 41.81) (end 73.14 28.13) (width 0.25) (layer F.Cu) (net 2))
 (segment (start 65 49.95) (end 73.14 41.81) (width 0.25) (layer F.Cu) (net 2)))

